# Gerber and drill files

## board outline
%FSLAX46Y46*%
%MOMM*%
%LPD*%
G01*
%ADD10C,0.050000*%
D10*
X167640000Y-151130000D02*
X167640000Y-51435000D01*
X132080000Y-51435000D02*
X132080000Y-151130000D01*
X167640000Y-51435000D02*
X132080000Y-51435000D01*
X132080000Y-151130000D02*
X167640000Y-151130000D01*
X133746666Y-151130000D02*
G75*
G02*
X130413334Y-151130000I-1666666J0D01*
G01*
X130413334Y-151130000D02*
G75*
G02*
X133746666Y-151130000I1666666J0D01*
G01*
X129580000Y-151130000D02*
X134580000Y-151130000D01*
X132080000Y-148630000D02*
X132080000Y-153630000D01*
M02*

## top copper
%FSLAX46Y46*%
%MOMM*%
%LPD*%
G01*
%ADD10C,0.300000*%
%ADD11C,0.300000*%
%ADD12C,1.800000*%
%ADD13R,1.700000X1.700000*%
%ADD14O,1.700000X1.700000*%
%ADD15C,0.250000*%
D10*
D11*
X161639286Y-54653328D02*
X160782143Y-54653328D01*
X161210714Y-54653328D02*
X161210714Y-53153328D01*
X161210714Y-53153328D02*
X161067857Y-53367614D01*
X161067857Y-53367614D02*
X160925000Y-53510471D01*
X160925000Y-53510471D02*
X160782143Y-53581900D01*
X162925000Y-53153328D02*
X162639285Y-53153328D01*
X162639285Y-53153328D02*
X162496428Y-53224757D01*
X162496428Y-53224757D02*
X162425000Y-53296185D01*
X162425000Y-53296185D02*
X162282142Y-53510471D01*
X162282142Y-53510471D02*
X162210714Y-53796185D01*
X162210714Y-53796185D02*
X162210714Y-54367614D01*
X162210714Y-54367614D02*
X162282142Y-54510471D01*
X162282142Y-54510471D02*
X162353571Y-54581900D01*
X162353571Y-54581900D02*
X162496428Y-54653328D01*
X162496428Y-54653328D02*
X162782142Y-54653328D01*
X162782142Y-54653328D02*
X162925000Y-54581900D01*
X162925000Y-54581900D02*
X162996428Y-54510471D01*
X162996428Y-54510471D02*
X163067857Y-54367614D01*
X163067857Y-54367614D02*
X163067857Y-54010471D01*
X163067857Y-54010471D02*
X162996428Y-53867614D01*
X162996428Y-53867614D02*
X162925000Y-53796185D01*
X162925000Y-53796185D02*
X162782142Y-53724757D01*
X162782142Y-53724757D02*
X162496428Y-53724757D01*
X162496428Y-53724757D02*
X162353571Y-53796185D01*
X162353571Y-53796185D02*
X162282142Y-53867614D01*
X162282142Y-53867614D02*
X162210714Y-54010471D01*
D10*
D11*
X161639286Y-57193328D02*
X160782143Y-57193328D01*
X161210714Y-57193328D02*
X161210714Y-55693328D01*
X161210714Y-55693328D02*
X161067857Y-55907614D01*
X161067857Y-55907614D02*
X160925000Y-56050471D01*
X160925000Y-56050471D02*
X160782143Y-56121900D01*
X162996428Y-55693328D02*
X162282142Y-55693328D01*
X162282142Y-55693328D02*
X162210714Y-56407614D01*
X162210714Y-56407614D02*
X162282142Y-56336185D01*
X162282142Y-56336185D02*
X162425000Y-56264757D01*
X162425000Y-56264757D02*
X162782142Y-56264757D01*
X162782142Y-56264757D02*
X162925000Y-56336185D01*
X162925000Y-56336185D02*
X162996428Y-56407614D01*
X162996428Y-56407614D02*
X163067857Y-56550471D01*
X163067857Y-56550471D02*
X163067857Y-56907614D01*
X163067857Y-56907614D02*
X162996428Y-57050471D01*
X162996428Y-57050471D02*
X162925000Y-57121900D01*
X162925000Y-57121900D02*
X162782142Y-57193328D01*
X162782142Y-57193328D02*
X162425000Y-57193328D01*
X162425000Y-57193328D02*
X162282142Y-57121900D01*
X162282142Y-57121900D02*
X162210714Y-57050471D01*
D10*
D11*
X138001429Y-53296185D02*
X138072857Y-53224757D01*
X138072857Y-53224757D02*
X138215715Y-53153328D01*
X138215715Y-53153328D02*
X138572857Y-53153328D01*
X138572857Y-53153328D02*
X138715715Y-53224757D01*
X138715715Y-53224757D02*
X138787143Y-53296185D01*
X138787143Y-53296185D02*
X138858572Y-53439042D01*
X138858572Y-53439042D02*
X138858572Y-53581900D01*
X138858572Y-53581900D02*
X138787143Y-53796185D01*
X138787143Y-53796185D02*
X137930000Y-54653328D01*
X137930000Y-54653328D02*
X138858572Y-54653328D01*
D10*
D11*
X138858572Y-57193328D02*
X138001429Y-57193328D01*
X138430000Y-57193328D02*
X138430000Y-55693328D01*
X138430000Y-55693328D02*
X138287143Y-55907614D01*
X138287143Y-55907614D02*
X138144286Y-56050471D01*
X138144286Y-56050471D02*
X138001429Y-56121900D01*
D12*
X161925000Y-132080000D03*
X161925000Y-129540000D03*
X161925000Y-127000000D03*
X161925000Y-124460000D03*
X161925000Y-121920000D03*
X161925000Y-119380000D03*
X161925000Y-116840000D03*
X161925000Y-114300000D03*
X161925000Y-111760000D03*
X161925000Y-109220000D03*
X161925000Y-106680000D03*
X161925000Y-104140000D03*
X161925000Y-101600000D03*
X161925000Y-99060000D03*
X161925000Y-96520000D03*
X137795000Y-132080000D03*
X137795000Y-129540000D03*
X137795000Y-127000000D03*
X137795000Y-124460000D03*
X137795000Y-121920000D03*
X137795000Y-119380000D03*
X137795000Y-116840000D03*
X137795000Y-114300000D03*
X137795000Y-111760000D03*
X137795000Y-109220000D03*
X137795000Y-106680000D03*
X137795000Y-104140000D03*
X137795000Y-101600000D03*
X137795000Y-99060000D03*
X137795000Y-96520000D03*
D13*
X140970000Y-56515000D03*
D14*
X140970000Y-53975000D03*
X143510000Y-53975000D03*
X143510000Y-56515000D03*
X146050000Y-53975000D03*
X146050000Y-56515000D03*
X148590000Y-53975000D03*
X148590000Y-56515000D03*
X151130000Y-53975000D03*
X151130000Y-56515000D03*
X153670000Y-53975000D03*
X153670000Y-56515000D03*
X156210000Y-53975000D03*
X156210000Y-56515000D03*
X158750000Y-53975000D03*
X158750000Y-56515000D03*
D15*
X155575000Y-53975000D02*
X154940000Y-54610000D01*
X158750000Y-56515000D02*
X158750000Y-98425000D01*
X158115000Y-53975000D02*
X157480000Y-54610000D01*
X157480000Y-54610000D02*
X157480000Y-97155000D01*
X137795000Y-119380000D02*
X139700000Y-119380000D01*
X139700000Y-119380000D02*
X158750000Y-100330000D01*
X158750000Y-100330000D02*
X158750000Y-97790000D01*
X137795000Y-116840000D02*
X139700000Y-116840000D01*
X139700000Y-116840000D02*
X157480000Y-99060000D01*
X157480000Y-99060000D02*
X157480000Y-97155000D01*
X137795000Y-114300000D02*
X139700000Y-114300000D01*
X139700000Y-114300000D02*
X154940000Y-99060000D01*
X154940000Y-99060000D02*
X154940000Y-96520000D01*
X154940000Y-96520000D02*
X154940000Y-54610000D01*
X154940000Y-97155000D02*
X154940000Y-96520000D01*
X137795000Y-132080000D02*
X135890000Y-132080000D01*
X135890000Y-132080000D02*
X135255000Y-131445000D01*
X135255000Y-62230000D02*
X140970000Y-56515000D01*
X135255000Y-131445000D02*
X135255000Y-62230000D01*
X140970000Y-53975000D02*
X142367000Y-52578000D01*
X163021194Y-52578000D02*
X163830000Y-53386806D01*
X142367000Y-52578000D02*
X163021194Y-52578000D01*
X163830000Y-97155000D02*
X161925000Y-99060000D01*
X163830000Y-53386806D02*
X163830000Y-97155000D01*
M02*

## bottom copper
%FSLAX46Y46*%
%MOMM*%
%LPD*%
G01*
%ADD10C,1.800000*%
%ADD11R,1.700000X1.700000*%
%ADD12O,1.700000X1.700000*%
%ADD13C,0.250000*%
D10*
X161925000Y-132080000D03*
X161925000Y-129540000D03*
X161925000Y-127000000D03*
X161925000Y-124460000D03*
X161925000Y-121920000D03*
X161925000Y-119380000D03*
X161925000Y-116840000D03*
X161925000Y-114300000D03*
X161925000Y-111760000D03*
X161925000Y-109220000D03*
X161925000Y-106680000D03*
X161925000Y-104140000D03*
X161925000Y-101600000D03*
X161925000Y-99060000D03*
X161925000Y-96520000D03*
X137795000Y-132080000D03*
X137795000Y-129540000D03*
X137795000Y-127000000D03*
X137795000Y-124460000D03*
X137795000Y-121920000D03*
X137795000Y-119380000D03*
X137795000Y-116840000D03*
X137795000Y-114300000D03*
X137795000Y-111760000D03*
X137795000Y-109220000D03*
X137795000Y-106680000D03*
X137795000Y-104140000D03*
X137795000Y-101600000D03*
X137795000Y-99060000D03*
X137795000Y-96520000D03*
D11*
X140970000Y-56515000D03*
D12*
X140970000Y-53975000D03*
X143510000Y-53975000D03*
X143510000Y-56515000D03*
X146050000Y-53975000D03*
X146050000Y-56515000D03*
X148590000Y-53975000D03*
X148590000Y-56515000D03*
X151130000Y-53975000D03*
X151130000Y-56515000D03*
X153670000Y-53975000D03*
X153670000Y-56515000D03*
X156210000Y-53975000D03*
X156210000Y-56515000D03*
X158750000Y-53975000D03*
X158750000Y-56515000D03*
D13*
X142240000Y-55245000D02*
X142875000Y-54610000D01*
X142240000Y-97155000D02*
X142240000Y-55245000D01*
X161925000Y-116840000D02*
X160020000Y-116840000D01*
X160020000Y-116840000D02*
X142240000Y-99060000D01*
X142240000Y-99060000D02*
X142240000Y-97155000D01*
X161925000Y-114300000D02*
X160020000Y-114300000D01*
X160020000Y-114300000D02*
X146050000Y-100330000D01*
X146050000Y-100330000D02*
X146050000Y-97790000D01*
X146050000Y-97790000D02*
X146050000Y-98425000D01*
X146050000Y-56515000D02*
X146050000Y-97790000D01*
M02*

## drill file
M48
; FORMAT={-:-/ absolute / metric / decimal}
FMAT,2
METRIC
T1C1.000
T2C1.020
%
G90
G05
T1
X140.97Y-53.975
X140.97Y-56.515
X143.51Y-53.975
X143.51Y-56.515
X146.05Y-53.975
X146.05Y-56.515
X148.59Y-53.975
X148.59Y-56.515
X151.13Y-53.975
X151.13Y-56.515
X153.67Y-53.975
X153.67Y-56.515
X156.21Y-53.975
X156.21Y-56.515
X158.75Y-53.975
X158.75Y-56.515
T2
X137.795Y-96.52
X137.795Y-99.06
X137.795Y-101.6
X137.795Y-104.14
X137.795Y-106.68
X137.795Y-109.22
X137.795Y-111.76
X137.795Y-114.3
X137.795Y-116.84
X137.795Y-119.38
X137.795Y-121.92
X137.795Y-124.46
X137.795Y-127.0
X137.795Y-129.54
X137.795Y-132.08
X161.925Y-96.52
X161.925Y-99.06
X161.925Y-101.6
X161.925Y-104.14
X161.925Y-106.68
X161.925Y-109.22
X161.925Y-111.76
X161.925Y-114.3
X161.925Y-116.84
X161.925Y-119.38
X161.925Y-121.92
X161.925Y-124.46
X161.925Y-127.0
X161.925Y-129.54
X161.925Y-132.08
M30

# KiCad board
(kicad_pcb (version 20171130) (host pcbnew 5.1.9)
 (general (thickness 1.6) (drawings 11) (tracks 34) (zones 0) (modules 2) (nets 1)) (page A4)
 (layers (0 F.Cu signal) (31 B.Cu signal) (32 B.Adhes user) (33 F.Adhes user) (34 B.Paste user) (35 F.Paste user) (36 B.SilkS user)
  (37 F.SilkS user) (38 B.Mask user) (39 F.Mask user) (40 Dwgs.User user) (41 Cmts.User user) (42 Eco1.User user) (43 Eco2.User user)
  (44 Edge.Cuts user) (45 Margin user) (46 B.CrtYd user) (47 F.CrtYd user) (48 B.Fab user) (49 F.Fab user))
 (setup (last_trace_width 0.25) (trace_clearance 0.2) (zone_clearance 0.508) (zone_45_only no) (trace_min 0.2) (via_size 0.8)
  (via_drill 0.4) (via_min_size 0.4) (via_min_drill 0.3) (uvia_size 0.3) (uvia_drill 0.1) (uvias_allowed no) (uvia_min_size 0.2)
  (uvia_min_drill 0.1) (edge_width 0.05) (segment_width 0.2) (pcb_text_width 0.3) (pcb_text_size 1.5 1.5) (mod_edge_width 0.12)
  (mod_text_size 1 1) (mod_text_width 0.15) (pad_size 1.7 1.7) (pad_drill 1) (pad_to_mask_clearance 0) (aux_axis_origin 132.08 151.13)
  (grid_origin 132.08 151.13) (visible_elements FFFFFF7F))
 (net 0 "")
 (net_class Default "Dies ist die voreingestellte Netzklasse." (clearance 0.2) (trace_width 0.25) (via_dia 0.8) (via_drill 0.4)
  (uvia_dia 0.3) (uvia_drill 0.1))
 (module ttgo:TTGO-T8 (layer F.Cu) (at 137.795 96.52)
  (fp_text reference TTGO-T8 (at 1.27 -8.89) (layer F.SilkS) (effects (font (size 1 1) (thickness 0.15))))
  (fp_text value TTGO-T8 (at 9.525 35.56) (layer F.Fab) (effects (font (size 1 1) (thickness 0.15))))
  (pad 5V thru_hole circle (at 24.13 35.56) (size 1.8 1.8) (drill 1.02) (layers *.Cu *.Mask))
  (pad 4 thru_hole circle (at 24.13 33.02) (size 1.8 1.8) (drill 1.02) (layers *.Cu *.Mask))
  (pad 0 thru_hole circle (at 24.13 30.48) (size 1.8 1.8) (drill 1.02) (layers *.Cu *.Mask))
  (pad GND thru_hole circle (at 24.13 27.94) (size 1.8 1.8) (drill 1.02) (layers *.Cu *.Mask))
  (pad 2 thru_hole circle (at 24.13 25.4) (size 1.8 1.8) (drill 1.02) (layers *.Cu *.Mask))
  (pad 5 thru_hole circle (at 24.13 22.86) (size 1.8 1.8) (drill 1.02) (layers *.Cu *.Mask))
  (pad 18 thru_hole circle (at 24.13 20.32) (size 1.8 1.8) (drill 1.02) (layers *.Cu *.Mask))
  (pad 23 thru_hole circle (at 24.13 17.78) (size 1.8 1.8) (drill 1.02) (layers *.Cu *.Mask))
  (pad 19 thru_hole circle (at 24.13 15.24) (size 1.8 1.8) (drill 1.02) (layers *.Cu *.Mask))
  (pad 22 thru_hole circle (at 24.13 12.7) (size 1.8 1.8) (drill 1.02) (layers *.Cu *.Mask))
  (pad RXD thru_hole circle (at 24.13 10.16) (size 1.8 1.8) (drill 1.02) (layers *.Cu *.Mask))
  (pad TXD thru_hole circle (at 24.13 7.62) (size 1.8 1.8) (drill 1.02) (layers *.Cu *.Mask))
  (pad 21 thru_hole circle (at 24.13 5.08) (size 1.8 1.8) (drill 1.02) (layers *.Cu *.Mask))
  (pad 3-3 thru_hole circle (at 24.13 2.54) (size 1.8 1.8) (drill 1.02) (layers *.Cu *.Mask))
  (pad GND thru_hole circle (at 24.13 0) (size 1.8 1.8) (drill 1.02) (layers *.Cu *.Mask))
  (pad GND thru_hole circle (at 0 35.56) (size 1.8 1.8) (drill 1.02) (layers *.Cu *.Mask))
  (pad 15 thru_hole circle (at 0 33.02) (size 1.8 1.8) (drill 1.02) (layers *.Cu *.Mask))
  (pad 13 thru_hole circle (at 0 30.48) (size 1.8 1.8) (drill 1.02) (layers *.Cu *.Mask))
  (pad 12 thru_hole circle (at 0 27.94) (size 1.8 1.8) (drill 1.02) (layers *.Cu *.Mask))
  (pad 14 thru_hole circle (at 0 25.4) (size 1.8 1.8) (drill 1.02) (layers *.Cu *.Mask))
  (pad 27 thru_hole circle (at 0 22.86) (size 1.8 1.8) (drill 1.02) (layers *.Cu *.Mask))
  (pad 26 thru_hole circle (at 0 20.32) (size 1.8 1.8) (drill 1.02) (layers *.Cu *.Mask))
  (pad 25 thru_hole circle (at 0 17.78) (size 1.8 1.8) (drill 1.02) (layers *.Cu *.Mask))
  (pad 33 thru_hole circle (at 0 15.24) (size 1.8 1.8) (drill 1.02) (layers *.Cu *.Mask))
  (pad 32 thru_hole circle (at 0 12.7) (size 1.8 1.8) (drill 1.02) (layers *.Cu *.Mask))
  (pad 35 thru_hole circle (at 0 10.16) (size 1.8 1.8) (drill 1.02) (layers *.Cu *.Mask))
  (pad 34 thru_hole circle (at 0 7.62) (size 1.8 1.8) (drill 1.02) (layers *.Cu *.Mask))
  (pad RST thru_hole circle (at 0 5.08) (size 1.8 1.8) (drill 1.02) (layers *.Cu *.Mask))
  (pad VN thru_hole circle (at 0 2.54) (size 1.8 1.8) (drill 1.02) (layers *.Cu *.Mask))
  (pad VP thru_hole circle (at 0 0) (size 1.8 1.8) (drill 1.02) (layers *.Cu *.Mask)))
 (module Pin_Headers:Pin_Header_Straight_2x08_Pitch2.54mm (layer B.Cu) (at 140.97 53.975 270)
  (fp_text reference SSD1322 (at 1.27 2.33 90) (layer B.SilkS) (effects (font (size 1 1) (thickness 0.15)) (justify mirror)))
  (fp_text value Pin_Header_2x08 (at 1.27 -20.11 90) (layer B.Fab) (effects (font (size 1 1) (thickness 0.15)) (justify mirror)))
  (pad 1 thru_hole rect (at 2.54 0 270) (size 1.7 1.7) (drill 1) (layers *.Cu *.Mask))
  (pad 2 thru_hole oval (at 0 0 270) (size 1.7 1.7) (drill 1) (layers *.Cu *.Mask))
  (pad 4 thru_hole oval (at 0 -2.54 270) (size 1.7 1.7) (drill 1) (layers *.Cu *.Mask))
  (pad 3 thru_hole oval (at 2.54 -2.54 270) (size 1.7 1.7) (drill 1) (layers *.Cu *.Mask))
  (pad 6 thru_hole oval (at 0 -5.08 270) (size 1.7 1.7) (drill 1) (layers *.Cu *.Mask))
  (pad 5 thru_hole oval (at 2.54 -5.08 270) (size 1.7 1.7) (drill 1) (layers *.Cu *.Mask))
  (pad 8 thru_hole oval (at 0 -7.62 270) (size 1.7 1.7) (drill 1) (layers *.Cu *.Mask))
  (pad 7 thru_hole oval (at 2.54 -7.62 270) (size 1.7 1.7) (drill 1) (layers *.Cu *.Mask))
  (pad 10 thru_hole oval (at 0 -10.16 270) (size 1.7 1.7) (drill 1) (layers *.Cu *.Mask))
  (pad 9 thru_hole oval (at 2.54 -10.16 270) (size 1.7 1.7) (drill 1) (layers *.Cu *.Mask))
  (pad 12 thru_hole oval (at 0 -12.7 270) (size 1.7 1.7) (drill 1) (layers *.Cu *.Mask))
  (pad 11 thru_hole oval (at 2.54 -12.7 270) (size 1.7 1.7) (drill 1) (layers *.Cu *.Mask))
  (pad 14 thru_hole oval (at 0 -15.24 270) (size 1.7 1.7) (drill 1) (layers *.Cu *.Mask))
  (pad 13 thru_hole oval (at 2.54 -15.24 270) (size 1.7 1.7) (drill 1) (layers *.Cu *.Mask))
  (pad 16 thru_hole oval (at 0 -17.78 270) (size 1.7 1.7) (drill 1) (layers *.Cu *.Mask))
  (pad 15 thru_hole oval (at 2.54 -17.78 270) (size 1.7 1.7) (drill 1) (layers *.Cu *.Mask)))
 (gr_line (start 167.64 151.13) (end 167.64 51.435) (layer Edge.Cuts) (width 0.05))
 (gr_line (start 132.08 51.435) (end 132.08 151.13) (layer Edge.Cuts) (width 0.05))
 (gr_line (start 167.64 51.435) (end 132.08 51.435) (layer Edge.Cuts) (width 0.05))
 (gr_line (start 132.08 151.13) (end 167.64 151.13) (layer Edge.Cuts) (width 0.05))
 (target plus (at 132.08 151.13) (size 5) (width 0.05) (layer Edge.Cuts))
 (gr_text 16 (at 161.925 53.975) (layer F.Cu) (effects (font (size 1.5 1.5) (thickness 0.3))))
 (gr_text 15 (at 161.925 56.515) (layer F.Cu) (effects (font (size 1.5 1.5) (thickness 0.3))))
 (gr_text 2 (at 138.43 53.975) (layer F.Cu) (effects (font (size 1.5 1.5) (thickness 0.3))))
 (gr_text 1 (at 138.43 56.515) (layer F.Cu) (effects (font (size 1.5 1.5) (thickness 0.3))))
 (segment (start 142.24 55.245) (end 142.875 54.61) (width 0.25) (layer B.Cu) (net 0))
 (segment (start 142.24 97.155) (end 142.24 55.245) (width 0.25) (layer B.Cu) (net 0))
 (segment (start 155.575 53.975) (end 154.94 54.61) (width 0.25) (layer F.Cu) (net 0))
 (segment (start 158.75 56.515) (end 158.75 98.425) (width 0.25) (layer F.Cu) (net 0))
 (segment (start 158.115 53.975) (end 157.48 54.61) (width 0.25) (layer F.Cu) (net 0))
 (segment (start 157.48 54.61) (end 157.48 97.155) (width 0.25) (layer F.Cu) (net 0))
 (segment (start 161.925 116.84) (end 160.02 116.84) (width 0.25) (layer B.Cu) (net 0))
 (segment (start 160.02 116.84) (end 142.24 99.06) (width 0.25) (layer B.Cu) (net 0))
 (segment (start 142.24 99.06) (end 142.24 97.155) (width 0.25) (layer B.Cu) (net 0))
 (segment (start 161.925 114.3) (end 160.02 114.3) (width 0.25) (layer B.Cu) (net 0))
 (segment (start 160.02 114.3) (end 146.05 100.33) (width 0.25) (layer B.Cu) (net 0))
 (segment (start 146.05 100.33) (end 146.05 97.79) (width 0.25) (layer B.Cu) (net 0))
 (segment (start 146.05 97.79) (end 146.05 98.425) (width 0.25) (layer B.Cu) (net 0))
 (segment (start 146.05 56.515) (end 146.05 97.79) (width 0.25) (layer B.Cu) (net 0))
 (segment (start 137.795 119.38) (end 139.7 119.38) (width 0.25) (layer F.Cu) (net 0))
 (segment (start 139.7 119.38) (end 158.75 100.33) (width 0.25) (layer F.Cu) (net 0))
 (segment (start 158.75 100.33) (end 158.75 97.79) (width 0.25) (layer F.Cu) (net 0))
 (segment (start 137.795 116.84) (end 139.7 116.84) (width 0.25) (layer F.Cu) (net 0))
 (segment (start 139.7 116.84) (end 157.48 99.06) (width 0.25) (layer F.Cu) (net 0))
 (segment (start 157.48 99.06) (end 157.48 97.155) (width 0.25) (layer F.Cu) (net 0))
 (segment (start 137.795 114.3) (end 139.7 114.3) (width 0.25) (layer F.Cu) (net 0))
 (segment (start 139.7 114.3) (end 154.94 99.06) (width 0.25) (layer F.Cu) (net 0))
 (segment (start 154.94 99.06) (end 154.94 96.52) (width 0.25) (layer F.Cu) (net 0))
 (segment (start 154.94 96.52) (end 154.94 54.61) (width 0.25) (layer F.Cu) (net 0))
 (segment (start 154.94 97.155) (end 154.94 96.52) (width 0.25) (layer F.Cu) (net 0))
 (segment (start 137.795 132.08) (end 135.89 132.08) (width 0.25) (layer F.Cu) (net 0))
 (segment (start 135.89 132.08) (end 135.255 131.445) (width 0.25) (layer F.Cu) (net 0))
 (segment (start 135.255 62.23) (end 140.97 56.515) (width 0.25) (layer F.Cu) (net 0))
 (segment (start 135.255 131.445) (end 135.255 62.23) (width 0.25) (layer F.Cu) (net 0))
 (segment (start 140.97 53.975) (end 142.367 52.578) (width 0.25) (layer F.Cu) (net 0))
 (segment (start 163.021194 52.578) (end 163.83 53.386806) (width 0.25) (layer F.Cu) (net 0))
 (segment (start 142.367 52.578) (end 163.021194 52.578) (width 0.25) (layer F.Cu) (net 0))
 (segment (start 163.83 97.155) (end 161.925 99.06) (width 0.25) (layer F.Cu) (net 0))
 (segment (start 163.83 53.386806) (end 163.83 97.155) (width 0.25) (layer F.Cu) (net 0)))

